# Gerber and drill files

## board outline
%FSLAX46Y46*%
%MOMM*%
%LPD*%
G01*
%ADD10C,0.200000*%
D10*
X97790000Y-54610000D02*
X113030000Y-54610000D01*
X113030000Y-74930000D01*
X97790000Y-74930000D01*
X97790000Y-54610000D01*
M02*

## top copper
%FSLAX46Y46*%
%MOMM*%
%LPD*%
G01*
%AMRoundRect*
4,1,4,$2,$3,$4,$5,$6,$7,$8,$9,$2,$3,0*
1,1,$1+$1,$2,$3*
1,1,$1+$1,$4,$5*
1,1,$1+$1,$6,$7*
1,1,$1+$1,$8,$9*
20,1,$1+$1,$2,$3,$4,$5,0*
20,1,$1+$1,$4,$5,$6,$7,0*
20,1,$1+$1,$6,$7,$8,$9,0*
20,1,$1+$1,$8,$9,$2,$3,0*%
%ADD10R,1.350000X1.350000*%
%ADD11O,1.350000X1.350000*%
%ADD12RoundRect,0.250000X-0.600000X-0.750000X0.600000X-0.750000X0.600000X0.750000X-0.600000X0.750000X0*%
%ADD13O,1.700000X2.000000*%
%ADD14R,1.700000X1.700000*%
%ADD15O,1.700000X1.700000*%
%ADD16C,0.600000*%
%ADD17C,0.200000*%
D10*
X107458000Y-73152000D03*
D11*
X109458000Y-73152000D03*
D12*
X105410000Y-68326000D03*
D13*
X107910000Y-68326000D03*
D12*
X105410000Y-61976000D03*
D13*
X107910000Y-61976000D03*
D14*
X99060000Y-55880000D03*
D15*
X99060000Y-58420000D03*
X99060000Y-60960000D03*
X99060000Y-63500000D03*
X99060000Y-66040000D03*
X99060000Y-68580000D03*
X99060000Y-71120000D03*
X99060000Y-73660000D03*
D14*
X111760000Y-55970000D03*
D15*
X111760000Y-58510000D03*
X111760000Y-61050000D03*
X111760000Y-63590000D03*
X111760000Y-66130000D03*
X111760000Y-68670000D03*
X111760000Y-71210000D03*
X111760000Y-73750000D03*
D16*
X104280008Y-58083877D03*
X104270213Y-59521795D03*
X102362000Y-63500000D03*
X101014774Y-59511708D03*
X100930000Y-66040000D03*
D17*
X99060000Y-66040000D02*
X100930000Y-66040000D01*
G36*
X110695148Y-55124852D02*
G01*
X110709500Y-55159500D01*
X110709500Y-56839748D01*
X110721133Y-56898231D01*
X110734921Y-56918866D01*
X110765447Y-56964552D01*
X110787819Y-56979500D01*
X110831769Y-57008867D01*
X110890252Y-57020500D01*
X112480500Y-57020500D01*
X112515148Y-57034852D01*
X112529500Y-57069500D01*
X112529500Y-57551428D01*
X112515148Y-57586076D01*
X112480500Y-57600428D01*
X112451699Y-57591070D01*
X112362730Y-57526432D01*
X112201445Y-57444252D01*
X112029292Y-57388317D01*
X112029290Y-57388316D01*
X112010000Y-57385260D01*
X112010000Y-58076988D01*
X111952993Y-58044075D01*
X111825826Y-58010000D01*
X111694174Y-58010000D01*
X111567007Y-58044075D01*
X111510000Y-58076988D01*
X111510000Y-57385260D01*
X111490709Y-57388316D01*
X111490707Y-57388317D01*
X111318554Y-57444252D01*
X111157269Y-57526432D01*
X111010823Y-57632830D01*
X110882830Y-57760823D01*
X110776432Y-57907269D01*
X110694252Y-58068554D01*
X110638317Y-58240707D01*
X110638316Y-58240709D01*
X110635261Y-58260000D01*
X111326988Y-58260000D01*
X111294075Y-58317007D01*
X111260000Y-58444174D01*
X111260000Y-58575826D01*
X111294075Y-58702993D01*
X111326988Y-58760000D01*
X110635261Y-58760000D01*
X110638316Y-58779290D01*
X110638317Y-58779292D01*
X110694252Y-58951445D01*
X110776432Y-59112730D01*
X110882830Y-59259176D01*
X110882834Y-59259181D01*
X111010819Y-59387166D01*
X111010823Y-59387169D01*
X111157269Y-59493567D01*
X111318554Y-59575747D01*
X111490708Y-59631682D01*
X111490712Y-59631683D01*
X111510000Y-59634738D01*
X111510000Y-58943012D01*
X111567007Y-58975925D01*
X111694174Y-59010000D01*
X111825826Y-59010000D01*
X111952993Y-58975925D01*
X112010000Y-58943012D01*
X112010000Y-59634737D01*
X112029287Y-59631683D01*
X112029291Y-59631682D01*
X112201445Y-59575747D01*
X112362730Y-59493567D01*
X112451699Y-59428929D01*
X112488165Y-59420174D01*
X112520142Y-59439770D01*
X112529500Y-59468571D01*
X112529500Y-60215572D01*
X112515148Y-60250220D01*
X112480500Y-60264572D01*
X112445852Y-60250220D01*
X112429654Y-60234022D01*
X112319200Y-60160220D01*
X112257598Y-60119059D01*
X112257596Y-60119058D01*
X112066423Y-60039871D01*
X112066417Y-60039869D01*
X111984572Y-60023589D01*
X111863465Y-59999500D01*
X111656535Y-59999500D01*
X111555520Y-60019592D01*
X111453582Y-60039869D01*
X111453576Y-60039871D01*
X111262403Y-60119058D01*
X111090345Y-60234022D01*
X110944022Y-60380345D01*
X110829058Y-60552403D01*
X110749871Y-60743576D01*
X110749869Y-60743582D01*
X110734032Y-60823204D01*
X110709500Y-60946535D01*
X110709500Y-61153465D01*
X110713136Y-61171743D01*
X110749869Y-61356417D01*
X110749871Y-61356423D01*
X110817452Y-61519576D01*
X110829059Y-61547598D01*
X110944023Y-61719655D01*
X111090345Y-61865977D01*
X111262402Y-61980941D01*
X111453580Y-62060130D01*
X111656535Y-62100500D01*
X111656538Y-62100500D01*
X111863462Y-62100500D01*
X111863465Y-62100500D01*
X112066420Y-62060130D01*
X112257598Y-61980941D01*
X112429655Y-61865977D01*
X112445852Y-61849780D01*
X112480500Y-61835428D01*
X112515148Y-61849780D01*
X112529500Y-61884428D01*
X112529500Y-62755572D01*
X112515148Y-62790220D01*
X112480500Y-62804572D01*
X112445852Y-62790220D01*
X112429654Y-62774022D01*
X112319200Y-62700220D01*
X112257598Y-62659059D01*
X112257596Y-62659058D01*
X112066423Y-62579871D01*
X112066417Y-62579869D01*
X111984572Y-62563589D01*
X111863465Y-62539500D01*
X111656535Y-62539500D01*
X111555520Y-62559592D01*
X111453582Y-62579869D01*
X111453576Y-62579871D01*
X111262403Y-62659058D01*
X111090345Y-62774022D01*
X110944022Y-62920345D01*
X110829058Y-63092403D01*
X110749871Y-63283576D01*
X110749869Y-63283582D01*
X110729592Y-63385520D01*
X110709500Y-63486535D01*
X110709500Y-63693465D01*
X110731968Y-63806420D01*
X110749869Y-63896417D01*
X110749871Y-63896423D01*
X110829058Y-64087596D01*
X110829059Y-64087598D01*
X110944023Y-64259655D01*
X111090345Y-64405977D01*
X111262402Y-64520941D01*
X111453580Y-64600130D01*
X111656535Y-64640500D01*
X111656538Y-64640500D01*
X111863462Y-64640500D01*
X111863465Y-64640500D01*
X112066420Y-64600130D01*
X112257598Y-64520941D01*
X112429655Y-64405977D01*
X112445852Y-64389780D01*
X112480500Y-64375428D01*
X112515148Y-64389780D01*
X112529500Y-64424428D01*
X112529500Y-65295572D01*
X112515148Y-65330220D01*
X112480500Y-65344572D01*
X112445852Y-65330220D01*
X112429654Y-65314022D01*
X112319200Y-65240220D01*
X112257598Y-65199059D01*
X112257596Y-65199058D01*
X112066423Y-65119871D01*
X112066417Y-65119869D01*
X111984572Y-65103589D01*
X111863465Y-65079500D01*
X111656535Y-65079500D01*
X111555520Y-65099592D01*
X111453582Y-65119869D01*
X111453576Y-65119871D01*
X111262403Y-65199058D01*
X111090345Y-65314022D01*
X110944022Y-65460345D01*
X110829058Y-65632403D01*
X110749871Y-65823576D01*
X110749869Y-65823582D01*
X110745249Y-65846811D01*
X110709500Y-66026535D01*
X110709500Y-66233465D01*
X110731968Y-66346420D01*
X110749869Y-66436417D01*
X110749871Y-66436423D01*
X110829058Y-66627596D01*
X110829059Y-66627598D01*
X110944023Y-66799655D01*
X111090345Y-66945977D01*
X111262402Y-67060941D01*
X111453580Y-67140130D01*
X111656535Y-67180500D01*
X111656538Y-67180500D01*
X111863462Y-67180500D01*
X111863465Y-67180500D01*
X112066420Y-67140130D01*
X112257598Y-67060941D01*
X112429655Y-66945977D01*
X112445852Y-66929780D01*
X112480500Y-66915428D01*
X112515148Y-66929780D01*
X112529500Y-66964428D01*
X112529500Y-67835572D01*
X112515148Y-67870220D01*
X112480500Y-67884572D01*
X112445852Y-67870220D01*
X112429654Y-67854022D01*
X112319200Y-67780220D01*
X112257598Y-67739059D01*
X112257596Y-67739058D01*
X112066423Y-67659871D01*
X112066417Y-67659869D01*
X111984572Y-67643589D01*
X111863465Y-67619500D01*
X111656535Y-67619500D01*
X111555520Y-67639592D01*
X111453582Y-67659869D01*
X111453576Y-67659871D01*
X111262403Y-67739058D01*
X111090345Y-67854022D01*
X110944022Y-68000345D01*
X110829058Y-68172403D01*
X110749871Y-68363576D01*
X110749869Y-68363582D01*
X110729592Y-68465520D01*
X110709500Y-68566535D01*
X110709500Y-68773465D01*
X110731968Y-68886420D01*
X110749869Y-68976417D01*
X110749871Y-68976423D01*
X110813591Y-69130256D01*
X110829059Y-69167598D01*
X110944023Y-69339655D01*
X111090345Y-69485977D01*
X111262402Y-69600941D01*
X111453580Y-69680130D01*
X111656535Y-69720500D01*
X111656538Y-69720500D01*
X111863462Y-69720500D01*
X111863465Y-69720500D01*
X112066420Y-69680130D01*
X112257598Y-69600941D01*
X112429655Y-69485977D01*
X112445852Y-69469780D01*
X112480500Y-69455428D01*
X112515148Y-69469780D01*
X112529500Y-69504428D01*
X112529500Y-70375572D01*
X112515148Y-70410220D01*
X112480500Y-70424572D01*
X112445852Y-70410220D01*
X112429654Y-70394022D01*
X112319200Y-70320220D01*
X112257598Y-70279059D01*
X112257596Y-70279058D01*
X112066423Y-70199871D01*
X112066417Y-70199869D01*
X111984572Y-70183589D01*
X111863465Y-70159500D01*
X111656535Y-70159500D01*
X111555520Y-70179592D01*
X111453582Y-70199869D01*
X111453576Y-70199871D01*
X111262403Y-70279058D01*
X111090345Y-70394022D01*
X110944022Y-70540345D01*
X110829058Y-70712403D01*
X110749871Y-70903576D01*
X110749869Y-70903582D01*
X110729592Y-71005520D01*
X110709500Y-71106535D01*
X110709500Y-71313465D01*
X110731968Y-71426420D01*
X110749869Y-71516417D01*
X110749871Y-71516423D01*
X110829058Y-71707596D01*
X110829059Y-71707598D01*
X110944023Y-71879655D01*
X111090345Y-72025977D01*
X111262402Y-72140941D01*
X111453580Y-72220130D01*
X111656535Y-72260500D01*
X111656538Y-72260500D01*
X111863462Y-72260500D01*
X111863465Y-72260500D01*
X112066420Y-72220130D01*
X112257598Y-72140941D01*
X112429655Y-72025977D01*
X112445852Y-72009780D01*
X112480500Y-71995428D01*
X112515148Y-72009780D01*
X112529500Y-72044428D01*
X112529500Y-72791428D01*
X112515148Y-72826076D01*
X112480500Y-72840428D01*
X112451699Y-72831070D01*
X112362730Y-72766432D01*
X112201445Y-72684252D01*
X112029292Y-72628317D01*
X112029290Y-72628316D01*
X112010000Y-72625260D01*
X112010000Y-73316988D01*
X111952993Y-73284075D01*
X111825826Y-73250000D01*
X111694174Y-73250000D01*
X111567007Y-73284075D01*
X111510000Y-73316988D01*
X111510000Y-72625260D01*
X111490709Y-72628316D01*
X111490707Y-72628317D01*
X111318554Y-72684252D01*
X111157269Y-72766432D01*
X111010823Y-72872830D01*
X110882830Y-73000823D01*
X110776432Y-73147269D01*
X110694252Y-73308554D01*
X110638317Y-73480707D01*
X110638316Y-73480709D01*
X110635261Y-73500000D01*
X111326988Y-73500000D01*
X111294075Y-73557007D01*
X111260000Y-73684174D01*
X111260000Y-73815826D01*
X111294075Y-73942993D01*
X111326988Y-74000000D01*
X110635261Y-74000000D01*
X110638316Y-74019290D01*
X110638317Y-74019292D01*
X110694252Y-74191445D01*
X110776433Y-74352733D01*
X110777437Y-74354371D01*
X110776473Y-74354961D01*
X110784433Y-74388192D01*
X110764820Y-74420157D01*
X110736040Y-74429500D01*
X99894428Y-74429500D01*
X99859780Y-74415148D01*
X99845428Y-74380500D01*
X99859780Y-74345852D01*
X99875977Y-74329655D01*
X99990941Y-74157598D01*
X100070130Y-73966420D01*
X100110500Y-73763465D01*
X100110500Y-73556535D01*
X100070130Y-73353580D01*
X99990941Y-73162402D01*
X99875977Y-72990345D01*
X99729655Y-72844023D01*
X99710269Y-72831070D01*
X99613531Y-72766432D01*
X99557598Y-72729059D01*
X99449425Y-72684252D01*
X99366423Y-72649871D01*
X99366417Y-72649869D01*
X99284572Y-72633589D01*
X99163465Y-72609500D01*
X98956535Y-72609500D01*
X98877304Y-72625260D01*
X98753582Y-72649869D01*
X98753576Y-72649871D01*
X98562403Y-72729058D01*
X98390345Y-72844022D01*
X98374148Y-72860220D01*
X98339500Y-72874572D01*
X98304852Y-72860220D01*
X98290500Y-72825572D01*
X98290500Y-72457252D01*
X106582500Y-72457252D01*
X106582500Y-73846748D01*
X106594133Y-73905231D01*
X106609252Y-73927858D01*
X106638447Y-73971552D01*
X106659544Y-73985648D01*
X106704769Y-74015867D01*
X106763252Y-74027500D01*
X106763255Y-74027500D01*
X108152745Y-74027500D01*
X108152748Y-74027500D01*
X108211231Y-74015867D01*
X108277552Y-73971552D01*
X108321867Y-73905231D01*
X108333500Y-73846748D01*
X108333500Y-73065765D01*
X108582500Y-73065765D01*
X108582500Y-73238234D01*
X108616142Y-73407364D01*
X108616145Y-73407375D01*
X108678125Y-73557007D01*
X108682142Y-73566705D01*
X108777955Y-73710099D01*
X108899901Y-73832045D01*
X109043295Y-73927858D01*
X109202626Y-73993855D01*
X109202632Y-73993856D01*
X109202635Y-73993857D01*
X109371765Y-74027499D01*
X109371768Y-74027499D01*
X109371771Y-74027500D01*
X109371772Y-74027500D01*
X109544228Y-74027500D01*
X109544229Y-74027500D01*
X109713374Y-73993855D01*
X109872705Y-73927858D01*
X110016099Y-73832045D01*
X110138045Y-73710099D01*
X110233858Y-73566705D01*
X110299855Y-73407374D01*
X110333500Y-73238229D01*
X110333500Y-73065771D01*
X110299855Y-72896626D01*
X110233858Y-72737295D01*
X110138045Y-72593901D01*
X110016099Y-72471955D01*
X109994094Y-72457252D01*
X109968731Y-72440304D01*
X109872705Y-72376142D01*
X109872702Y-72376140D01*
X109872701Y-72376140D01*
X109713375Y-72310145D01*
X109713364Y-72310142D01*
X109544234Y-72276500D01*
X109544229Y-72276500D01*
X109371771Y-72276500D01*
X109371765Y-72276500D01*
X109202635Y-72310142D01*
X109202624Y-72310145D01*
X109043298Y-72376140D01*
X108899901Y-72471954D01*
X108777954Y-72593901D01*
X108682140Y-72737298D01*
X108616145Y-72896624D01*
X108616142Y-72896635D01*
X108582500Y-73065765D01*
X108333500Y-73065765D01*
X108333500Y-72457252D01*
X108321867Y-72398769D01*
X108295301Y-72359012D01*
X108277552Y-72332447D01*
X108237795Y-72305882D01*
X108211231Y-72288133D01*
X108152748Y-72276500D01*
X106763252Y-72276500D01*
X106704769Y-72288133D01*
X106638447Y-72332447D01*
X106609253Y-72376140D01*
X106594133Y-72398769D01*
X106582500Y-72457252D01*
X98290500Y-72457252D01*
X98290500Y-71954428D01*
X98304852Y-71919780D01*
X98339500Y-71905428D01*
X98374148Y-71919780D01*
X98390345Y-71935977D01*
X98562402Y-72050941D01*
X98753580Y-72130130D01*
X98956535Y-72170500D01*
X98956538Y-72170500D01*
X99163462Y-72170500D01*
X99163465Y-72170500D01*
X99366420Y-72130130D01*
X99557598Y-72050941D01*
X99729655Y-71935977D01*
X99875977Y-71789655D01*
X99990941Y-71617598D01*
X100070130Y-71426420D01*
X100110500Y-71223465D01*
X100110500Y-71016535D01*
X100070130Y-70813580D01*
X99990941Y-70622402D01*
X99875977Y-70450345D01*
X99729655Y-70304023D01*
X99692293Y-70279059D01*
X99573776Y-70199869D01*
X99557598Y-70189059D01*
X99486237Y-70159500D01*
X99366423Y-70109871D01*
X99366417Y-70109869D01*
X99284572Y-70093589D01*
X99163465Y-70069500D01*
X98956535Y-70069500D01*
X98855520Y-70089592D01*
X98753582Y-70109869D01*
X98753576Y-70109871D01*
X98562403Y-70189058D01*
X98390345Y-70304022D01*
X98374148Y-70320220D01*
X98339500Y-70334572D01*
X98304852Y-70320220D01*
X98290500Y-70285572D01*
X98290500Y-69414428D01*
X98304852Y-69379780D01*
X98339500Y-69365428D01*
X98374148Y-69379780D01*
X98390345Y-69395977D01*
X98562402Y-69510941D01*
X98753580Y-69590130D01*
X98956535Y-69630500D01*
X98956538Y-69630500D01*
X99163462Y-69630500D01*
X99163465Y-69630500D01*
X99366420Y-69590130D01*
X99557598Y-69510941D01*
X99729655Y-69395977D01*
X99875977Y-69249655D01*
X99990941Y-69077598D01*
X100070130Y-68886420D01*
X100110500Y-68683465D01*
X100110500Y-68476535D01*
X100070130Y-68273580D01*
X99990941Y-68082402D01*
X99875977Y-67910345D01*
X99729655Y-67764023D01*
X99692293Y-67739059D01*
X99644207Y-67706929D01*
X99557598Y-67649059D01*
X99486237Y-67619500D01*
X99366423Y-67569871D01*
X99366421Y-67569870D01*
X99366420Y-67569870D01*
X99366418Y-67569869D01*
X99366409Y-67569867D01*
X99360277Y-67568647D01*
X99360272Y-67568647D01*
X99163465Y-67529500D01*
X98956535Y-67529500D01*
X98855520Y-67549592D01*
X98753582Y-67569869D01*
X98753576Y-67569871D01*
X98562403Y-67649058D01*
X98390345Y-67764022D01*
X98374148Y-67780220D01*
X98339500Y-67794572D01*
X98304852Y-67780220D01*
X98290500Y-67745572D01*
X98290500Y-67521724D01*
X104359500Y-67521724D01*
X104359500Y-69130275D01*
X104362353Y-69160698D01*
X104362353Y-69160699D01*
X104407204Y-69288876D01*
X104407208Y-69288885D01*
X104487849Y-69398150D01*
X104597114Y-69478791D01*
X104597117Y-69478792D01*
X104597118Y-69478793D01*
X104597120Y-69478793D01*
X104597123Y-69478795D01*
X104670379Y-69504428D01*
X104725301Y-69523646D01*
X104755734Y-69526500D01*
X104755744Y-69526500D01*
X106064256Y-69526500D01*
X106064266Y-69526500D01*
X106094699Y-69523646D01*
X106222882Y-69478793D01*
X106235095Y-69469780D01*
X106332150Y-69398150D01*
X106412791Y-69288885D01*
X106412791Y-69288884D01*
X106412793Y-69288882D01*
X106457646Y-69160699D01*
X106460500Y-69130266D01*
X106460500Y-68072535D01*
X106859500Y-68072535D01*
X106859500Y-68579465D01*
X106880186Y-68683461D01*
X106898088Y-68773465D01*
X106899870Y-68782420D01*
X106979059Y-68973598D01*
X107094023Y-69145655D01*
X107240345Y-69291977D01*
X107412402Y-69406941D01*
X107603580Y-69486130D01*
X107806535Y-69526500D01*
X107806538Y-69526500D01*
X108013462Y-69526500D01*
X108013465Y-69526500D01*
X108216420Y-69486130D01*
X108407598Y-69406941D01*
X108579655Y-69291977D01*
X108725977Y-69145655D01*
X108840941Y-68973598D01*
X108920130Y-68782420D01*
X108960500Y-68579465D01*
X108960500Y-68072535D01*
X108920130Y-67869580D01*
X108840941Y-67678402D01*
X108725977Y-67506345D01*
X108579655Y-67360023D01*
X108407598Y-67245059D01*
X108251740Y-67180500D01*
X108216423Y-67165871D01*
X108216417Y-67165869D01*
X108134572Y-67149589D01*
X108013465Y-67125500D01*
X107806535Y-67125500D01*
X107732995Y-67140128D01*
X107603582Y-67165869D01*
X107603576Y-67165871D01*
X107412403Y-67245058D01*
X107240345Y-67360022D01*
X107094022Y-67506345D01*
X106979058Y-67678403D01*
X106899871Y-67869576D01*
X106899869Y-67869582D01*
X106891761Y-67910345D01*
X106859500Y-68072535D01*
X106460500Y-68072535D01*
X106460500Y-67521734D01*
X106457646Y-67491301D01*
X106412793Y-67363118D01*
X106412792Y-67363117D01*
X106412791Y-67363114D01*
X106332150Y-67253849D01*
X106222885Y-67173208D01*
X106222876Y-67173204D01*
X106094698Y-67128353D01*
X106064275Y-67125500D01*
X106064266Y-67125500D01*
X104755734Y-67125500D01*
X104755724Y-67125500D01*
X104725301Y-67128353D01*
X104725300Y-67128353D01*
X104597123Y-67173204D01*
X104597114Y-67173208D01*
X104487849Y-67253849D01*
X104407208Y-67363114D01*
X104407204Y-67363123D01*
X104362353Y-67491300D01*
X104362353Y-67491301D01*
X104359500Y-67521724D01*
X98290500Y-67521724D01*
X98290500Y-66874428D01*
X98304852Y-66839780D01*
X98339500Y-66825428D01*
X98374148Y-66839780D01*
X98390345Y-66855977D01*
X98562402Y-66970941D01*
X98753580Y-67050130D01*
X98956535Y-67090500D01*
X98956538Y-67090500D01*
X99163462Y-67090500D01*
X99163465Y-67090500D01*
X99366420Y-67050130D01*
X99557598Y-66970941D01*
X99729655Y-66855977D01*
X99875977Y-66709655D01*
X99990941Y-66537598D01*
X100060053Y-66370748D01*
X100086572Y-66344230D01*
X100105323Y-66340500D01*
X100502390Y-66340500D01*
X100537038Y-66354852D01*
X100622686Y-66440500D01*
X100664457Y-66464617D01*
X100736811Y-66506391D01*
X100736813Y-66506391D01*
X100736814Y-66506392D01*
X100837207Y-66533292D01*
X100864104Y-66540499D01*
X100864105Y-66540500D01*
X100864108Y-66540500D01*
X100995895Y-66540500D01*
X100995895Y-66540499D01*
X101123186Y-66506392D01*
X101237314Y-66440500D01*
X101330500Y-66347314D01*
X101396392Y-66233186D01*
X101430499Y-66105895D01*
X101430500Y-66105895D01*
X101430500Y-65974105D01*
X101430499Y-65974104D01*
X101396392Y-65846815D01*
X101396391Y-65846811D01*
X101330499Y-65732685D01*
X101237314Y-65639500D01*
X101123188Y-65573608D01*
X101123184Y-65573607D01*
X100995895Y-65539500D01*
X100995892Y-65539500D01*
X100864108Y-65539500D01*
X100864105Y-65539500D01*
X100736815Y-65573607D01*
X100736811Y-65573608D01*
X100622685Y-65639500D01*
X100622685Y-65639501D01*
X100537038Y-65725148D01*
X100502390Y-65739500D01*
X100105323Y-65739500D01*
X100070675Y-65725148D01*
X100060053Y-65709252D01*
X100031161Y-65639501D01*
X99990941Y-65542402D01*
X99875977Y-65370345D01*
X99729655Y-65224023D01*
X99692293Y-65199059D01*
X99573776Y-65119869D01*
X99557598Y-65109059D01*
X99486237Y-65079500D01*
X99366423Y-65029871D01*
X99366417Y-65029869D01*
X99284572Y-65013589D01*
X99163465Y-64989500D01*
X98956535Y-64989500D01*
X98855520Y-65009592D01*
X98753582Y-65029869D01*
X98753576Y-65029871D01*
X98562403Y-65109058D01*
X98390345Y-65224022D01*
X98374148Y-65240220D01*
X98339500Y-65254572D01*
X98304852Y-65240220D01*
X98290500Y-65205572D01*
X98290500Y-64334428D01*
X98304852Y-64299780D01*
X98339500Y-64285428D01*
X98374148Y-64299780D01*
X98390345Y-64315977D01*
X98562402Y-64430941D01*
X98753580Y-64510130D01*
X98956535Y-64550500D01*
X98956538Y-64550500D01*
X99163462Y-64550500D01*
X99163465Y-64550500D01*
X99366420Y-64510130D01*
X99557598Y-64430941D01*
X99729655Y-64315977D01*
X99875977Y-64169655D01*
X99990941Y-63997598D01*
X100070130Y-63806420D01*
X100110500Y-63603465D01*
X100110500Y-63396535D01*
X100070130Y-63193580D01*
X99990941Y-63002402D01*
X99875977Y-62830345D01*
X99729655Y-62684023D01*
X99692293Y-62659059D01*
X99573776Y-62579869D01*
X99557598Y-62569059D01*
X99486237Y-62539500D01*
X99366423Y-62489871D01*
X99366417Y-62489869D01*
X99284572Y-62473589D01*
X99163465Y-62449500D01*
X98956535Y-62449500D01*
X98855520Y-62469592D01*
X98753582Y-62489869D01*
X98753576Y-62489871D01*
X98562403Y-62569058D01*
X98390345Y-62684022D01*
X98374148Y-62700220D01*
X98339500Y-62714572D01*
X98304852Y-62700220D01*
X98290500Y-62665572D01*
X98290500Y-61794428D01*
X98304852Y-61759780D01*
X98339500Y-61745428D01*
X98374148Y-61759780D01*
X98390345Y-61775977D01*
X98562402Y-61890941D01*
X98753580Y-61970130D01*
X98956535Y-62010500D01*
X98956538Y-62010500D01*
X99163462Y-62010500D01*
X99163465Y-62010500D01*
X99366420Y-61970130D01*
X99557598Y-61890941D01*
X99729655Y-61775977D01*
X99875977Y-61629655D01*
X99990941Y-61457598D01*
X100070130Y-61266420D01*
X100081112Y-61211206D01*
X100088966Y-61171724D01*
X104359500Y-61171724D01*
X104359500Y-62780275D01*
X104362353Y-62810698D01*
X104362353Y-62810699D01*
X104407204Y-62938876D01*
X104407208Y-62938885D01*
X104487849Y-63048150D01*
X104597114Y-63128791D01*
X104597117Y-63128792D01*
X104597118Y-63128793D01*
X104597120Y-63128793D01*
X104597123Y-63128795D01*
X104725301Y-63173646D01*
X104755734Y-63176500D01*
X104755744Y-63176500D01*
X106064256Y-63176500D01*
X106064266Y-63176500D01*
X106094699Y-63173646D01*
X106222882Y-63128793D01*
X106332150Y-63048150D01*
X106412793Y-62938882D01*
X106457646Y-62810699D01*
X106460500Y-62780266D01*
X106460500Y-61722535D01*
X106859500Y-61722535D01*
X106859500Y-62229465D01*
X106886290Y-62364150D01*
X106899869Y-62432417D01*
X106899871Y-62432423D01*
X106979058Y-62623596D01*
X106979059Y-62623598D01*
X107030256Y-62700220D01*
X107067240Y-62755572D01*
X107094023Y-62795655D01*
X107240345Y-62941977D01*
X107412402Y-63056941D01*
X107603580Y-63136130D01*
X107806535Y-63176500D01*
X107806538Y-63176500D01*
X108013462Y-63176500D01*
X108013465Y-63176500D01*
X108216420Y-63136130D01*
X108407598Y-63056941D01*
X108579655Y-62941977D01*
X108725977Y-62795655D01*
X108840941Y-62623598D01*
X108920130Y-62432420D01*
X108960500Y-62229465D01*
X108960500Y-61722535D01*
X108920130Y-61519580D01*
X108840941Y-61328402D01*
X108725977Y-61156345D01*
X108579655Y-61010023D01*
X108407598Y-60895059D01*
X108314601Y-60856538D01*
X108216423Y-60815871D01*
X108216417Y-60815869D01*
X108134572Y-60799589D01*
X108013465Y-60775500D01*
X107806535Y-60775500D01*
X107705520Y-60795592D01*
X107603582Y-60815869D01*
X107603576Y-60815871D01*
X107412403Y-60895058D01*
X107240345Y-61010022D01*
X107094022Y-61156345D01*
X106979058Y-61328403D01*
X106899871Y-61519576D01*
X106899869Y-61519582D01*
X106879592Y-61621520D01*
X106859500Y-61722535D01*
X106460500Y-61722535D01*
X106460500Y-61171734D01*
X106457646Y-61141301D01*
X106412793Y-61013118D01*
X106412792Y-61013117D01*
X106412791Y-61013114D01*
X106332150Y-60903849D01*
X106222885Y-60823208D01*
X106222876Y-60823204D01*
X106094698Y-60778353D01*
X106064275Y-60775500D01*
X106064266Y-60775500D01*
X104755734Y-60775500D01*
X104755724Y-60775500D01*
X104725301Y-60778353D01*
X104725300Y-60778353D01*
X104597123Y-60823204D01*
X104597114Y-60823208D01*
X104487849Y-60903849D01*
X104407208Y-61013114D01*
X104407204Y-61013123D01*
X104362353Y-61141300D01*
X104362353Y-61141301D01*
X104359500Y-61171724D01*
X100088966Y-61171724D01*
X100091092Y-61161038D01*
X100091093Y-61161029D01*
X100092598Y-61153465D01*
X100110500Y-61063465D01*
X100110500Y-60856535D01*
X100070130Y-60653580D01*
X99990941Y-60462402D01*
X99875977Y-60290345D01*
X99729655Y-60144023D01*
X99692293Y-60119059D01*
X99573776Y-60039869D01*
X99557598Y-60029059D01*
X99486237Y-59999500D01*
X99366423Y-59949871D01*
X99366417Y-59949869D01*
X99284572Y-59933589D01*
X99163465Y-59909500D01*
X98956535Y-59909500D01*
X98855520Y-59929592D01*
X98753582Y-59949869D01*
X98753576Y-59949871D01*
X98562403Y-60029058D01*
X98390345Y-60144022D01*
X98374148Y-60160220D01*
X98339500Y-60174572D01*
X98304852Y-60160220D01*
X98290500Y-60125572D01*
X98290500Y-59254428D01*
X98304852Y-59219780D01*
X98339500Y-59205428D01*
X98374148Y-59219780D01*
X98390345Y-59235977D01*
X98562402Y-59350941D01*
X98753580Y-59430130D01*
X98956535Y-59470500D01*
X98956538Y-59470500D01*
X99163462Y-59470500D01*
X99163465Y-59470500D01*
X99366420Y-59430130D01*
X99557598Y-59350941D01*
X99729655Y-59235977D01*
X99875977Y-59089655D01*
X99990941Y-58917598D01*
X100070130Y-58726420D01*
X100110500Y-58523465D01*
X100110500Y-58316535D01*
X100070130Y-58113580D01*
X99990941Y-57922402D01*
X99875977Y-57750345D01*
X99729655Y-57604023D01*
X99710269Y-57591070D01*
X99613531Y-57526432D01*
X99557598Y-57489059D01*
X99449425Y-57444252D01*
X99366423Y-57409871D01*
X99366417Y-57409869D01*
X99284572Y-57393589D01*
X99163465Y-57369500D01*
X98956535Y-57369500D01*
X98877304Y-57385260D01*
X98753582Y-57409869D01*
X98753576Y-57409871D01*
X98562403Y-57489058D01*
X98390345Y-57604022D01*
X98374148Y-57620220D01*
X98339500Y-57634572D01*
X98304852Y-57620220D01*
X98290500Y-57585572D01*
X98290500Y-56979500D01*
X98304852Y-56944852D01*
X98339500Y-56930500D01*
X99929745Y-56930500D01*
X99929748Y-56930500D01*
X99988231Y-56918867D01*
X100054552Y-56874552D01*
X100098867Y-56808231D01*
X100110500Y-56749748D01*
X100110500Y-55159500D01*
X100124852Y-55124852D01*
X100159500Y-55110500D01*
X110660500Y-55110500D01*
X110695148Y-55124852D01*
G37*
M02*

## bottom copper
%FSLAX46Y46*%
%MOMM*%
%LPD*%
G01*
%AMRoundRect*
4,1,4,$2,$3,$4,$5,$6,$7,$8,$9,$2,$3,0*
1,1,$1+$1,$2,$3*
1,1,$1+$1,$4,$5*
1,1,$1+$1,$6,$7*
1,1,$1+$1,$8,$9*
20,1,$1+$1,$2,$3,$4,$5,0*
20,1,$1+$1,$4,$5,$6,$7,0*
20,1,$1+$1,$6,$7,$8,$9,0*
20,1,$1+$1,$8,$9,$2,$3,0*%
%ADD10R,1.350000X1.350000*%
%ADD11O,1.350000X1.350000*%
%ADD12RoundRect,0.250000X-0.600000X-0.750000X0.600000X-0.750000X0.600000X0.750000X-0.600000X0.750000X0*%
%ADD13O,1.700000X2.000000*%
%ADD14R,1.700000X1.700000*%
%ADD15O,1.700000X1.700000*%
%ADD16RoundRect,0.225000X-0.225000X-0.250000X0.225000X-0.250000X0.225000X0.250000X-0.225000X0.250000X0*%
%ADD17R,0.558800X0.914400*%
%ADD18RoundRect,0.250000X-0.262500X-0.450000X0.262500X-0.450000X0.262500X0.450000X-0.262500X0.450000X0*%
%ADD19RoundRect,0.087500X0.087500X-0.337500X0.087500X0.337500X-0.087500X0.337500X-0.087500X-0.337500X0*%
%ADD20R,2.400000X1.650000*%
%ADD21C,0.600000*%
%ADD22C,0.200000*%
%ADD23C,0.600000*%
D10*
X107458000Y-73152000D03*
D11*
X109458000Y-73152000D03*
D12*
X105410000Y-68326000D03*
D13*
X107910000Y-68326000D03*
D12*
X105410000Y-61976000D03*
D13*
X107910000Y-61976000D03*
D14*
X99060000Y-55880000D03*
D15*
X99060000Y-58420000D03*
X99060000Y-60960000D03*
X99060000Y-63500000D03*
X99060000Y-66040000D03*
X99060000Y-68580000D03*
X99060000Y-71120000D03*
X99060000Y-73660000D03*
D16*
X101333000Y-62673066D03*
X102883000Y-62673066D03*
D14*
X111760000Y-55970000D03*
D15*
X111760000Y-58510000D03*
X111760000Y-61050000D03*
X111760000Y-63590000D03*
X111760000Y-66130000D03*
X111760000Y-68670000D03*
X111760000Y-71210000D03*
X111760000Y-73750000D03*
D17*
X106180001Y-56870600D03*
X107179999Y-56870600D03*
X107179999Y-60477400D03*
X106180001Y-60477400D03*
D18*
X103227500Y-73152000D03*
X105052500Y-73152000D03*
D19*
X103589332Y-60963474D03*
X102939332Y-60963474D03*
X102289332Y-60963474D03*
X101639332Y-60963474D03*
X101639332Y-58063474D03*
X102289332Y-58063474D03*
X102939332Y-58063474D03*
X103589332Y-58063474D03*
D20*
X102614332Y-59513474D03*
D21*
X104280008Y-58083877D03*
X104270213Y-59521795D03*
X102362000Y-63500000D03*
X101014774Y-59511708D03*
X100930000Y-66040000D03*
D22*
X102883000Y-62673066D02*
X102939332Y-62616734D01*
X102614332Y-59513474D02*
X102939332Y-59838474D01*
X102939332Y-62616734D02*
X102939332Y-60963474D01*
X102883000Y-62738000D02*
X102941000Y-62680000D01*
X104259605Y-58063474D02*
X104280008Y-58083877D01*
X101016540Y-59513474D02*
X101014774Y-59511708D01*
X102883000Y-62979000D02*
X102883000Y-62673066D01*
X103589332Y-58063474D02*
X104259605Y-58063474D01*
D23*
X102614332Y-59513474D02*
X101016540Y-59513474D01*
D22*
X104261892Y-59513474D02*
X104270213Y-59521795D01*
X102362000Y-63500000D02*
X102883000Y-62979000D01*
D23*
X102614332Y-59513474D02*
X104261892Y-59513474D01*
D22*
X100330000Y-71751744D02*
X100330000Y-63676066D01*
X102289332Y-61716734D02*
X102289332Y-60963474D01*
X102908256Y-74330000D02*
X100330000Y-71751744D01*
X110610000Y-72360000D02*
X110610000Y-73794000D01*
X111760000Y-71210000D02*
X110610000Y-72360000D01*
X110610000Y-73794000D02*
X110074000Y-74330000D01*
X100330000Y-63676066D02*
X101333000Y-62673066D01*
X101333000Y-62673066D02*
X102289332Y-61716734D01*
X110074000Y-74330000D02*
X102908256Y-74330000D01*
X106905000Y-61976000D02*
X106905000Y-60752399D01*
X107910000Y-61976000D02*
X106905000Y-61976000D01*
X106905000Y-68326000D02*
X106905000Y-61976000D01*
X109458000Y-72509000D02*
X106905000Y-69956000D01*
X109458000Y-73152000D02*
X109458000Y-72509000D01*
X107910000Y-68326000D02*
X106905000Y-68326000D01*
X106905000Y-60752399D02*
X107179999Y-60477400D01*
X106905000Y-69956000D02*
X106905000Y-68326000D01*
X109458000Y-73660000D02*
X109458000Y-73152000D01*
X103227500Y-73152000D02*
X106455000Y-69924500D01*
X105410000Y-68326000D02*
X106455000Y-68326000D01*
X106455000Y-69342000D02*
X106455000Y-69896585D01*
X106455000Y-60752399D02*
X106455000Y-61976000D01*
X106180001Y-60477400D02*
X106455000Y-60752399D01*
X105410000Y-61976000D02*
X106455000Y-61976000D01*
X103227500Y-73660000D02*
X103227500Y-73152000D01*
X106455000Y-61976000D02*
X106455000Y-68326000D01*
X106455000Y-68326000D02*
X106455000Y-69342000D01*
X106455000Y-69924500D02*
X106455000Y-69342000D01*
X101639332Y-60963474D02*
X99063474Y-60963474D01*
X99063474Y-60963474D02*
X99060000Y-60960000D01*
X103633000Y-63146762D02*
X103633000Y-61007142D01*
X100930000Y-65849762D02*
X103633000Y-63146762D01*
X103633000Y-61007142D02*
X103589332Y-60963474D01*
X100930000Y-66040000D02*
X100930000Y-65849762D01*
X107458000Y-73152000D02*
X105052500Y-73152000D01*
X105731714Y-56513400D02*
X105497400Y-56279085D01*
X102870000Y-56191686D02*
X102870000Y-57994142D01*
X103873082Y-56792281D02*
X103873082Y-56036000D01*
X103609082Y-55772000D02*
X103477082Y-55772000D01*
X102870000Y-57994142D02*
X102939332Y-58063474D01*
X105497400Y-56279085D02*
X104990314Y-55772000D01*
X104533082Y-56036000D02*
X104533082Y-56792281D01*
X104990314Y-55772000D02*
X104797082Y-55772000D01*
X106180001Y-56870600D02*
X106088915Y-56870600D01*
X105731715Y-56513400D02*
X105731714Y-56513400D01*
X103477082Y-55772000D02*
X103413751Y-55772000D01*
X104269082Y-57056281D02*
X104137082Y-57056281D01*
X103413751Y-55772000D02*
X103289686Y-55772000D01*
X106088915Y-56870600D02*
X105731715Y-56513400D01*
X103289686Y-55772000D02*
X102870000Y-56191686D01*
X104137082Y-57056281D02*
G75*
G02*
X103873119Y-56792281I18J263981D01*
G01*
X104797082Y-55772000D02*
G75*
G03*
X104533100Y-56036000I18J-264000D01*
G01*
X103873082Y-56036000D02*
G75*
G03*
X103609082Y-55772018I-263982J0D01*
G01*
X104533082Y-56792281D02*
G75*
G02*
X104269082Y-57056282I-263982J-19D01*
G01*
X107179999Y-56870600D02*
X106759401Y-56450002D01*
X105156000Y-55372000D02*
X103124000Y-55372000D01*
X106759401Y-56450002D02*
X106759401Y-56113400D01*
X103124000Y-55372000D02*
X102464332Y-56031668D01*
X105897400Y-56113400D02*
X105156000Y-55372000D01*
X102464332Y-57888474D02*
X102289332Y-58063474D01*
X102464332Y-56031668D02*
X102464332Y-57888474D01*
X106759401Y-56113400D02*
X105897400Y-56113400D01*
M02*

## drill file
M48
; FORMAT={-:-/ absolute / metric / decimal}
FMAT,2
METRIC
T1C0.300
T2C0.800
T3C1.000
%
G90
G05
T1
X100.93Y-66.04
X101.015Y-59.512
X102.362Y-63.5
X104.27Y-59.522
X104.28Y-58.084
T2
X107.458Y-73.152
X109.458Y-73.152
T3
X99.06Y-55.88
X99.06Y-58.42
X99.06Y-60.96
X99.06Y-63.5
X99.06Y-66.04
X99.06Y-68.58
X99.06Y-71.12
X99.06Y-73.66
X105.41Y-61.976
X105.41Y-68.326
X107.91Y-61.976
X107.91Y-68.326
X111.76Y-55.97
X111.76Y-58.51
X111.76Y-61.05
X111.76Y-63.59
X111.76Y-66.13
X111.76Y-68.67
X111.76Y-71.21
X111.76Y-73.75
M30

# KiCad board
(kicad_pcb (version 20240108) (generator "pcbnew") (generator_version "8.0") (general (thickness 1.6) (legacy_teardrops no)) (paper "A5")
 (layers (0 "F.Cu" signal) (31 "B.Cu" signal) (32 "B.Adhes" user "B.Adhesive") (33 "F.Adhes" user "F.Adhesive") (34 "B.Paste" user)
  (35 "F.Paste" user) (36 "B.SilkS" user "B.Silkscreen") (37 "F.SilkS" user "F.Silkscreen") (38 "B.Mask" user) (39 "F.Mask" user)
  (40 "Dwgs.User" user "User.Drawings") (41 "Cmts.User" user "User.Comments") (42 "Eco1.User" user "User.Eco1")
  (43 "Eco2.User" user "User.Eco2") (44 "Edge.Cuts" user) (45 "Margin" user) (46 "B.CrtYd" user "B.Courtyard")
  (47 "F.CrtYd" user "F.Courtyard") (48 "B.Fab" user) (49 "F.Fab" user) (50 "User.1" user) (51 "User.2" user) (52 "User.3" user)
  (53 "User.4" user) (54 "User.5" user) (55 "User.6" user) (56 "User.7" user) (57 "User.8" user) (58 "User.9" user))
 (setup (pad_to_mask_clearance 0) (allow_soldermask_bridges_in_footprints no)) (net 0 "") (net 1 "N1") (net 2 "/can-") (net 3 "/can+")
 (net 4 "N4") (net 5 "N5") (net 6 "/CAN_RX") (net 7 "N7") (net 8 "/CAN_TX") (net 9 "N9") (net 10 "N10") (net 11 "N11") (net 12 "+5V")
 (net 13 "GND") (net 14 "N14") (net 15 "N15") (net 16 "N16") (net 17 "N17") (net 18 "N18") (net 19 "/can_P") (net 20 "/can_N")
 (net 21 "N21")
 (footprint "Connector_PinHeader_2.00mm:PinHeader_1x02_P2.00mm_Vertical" (layer "F.Cu") (at 107.458 73.152 90)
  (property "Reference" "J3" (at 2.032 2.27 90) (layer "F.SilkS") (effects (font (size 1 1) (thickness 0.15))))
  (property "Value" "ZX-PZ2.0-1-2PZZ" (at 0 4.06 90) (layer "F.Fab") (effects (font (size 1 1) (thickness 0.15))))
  (pad "1" thru_hole rect (at 0 0 90) (size 1.35 1.35) (drill 0.8) (layers "*.Cu" "*.Mask") (remove_unused_layers no) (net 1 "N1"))
  (pad "2" thru_hole oval (at 0 2 90) (size 1.35 1.35) (drill 0.8) (layers "*.Cu" "*.Mask") (remove_unused_layers no) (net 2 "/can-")))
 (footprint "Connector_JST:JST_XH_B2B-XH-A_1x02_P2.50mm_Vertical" (layer "F.Cu") (at 105.41 68.326)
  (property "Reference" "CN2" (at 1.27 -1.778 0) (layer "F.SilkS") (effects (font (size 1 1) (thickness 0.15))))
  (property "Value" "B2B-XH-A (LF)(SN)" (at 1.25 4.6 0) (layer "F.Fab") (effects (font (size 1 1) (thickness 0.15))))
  (pad "1" thru_hole roundrect (at 0 0) (size 1.7 2) (drill 1) (layers "*.Cu" "*.Mask") (remove_unused_layers no)
   (roundrect_rratio 0.147059) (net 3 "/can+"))
  (pad "2" thru_hole oval (at 2.5 0) (size 1.7 2) (drill 1) (layers "*.Cu" "*.Mask") (remove_unused_layers no) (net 2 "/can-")))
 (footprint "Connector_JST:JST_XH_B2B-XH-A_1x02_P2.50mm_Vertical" (layer "F.Cu") (at 105.41 61.976)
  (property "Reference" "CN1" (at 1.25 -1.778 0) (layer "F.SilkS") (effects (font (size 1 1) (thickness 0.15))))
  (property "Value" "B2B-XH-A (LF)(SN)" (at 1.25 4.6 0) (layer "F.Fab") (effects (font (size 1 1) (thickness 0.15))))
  (pad "1" thru_hole roundrect (at 0 0) (size 1.7 2) (drill 1) (layers "*.Cu" "*.Mask") (remove_unused_layers no)
   (roundrect_rratio 0.147059) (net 3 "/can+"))
  (pad "2" thru_hole oval (at 2.5 0) (size 1.7 2) (drill 1) (layers "*.Cu" "*.Mask") (remove_unused_layers no) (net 2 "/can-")))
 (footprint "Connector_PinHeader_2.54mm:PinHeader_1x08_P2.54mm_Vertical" (layer "B.Cu") (at 99.06 55.88 180)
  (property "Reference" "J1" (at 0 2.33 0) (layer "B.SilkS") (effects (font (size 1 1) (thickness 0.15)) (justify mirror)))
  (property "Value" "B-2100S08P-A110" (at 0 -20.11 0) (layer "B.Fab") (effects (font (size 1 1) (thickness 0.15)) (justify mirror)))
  (pad "1" thru_hole rect (at 0 0 180) (size 1.7 1.7) (drill 1) (layers "*.Cu" "*.Mask") (remove_unused_layers no) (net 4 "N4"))
  (pad "2" thru_hole oval (at 0 -2.54 180) (size 1.7 1.7) (drill 1) (layers "*.Cu" "*.Mask") (remove_unused_layers no) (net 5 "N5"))
  (pad "3" thru_hole oval (at 0 -5.08 180) (size 1.7 1.7) (drill 1) (layers "*.Cu" "*.Mask") (remove_unused_layers no) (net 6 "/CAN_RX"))
  (pad "4" thru_hole oval (at 0 -7.62 180) (size 1.7 1.7) (drill 1) (layers "*.Cu" "*.Mask") (remove_unused_layers no) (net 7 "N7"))
  (pad "5" thru_hole oval (at 0 -10.16 180) (size 1.7 1.7) (drill 1) (layers "*.Cu" "*.Mask") (remove_unused_layers no) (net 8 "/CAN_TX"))
  (pad "6" thru_hole oval (at 0 -12.7 180) (size 1.7 1.7) (drill 1) (layers "*.Cu" "*.Mask") (remove_unused_layers no) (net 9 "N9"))
  (pad "7" thru_hole oval (at 0 -15.24 180) (size 1.7 1.7) (drill 1) (layers "*.Cu" "*.Mask") (remove_unused_layers no) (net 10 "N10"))
  (pad "8" thru_hole oval (at 0 -17.78 180) (size 1.7 1.7) (drill 1) (layers "*.Cu" "*.Mask") (remove_unused_layers no) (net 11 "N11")))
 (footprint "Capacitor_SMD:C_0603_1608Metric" (layer "B.Cu") (at 102.108 62.673066)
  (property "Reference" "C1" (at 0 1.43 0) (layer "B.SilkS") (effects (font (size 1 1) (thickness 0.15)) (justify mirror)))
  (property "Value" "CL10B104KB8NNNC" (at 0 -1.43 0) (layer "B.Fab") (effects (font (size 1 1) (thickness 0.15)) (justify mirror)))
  (pad "1" smd roundrect (at -0.775 0) (size 0.9 0.95) (layers "B.Cu" "B.Paste" "B.Mask") (roundrect_rratio 0.25) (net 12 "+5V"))
  (pad "2" smd roundrect (at 0.775 0) (size 0.9 0.95) (layers "B.Cu" "B.Paste" "B.Mask") (roundrect_rratio 0.25) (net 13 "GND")))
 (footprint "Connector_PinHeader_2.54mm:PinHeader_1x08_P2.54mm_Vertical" (layer "B.Cu") (at 111.76 55.97 180)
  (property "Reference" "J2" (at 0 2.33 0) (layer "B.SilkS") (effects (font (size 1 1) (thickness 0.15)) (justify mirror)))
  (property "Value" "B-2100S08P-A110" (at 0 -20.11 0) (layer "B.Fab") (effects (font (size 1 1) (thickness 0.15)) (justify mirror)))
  (pad "1" thru_hole rect (at 0 0 180) (size 1.7 1.7) (drill 1) (layers "*.Cu" "*.Mask") (remove_unused_layers no) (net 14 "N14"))
  (pad "2" thru_hole oval (at 0 -2.54 180) (size 1.7 1.7) (drill 1) (layers "*.Cu" "*.Mask") (remove_unused_layers no) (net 13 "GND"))
  (pad "3" thru_hole oval (at 0 -5.08 180) (size 1.7 1.7) (drill 1) (layers "*.Cu" "*.Mask") (remove_unused_layers no) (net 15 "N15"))
  (pad "4" thru_hole oval (at 0 -7.62 180) (size 1.7 1.7) (drill 1) (layers "*.Cu" "*.Mask") (remove_unused_layers no) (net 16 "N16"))
  (pad "5" thru_hole oval (at 0 -10.16 180) (size 1.7 1.7) (drill 1) (layers "*.Cu" "*.Mask") (remove_unused_layers no) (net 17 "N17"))
  (pad "6" thru_hole oval (at 0 -12.7 180) (size 1.7 1.7) (drill 1) (layers "*.Cu" "*.Mask") (remove_unused_layers no) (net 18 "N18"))
  (pad "7" thru_hole oval (at 0 -15.24 180) (size 1.7 1.7) (drill 1) (layers "*.Cu" "*.Mask") (remove_unused_layers no) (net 12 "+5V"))
  (pad "8" thru_hole oval (at 0 -17.78 180) (size 1.7 1.7) (drill 1) (layers "*.Cu" "*.Mask") (remove_unused_layers no) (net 13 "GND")))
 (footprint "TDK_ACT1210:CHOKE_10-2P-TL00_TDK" (layer "B.Cu") (at 106.68 58.674 -90)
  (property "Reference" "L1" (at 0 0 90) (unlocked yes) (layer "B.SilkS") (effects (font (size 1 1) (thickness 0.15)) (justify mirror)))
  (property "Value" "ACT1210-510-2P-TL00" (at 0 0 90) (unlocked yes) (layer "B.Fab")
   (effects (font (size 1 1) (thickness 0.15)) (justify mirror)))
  (pad "1" smd rect (at -1.8034 0.499999 270) (size 0.9144 0.5588) (layers "B.Cu" "B.Paste" "B.Mask") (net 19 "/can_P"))
  (pad "2" smd rect (at -1.8034 -0.499999 270) (size 0.9144 0.5588) (layers "B.Cu" "B.Paste" "B.Mask") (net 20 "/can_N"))
  (pad "3" smd rect (at 1.8034 -0.499999 270) (size 0.9144 0.5588) (layers "B.Cu" "B.Paste" "B.Mask") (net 2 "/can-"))
  (pad "4" smd rect (at 1.8034 0.499999 270) (size 0.9144 0.5588) (layers "B.Cu" "B.Paste" "B.Mask") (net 3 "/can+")))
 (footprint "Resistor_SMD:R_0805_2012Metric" (layer "B.Cu") (at 104.14 73.152)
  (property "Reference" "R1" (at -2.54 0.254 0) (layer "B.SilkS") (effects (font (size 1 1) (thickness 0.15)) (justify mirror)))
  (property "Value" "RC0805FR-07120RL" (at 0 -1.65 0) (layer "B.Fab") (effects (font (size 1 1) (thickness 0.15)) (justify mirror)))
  (pad "1" smd roundrect (at -0.9125 0) (size 1.025 1.4) (layers "B.Cu" "B.Paste" "B.Mask") (roundrect_rratio 0.243902) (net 3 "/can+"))
  (pad "2" smd roundrect (at 0.9125 0) (size 1.025 1.4) (layers "B.Cu" "B.Paste" "B.Mask") (roundrect_rratio 0.243902) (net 1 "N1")))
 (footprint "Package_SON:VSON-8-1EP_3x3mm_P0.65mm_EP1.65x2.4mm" (layer "B.Cu") (at 102.614332 59.513474 90)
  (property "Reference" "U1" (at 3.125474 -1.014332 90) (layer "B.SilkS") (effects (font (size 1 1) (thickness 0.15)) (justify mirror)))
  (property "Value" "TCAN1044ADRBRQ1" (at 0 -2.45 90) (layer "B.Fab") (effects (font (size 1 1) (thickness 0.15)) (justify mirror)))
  (pad "" smd roundrect (at 0 0 90) (size 1.33 1.93) (layers "B.Paste") (roundrect_rratio 0.18797))
  (pad "1" smd roundrect (at -1.45 0.975 90) (size 0.85 0.35) (layers "B.Cu" "B.Paste" "B.Mask") (roundrect_rratio 0.25) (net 8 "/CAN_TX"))
  (pad "2" smd roundrect (at -1.45 0.325 90) (size 0.85 0.35) (layers "B.Cu" "B.Paste" "B.Mask") (roundrect_rratio 0.25) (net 13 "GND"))
  (pad "3" smd roundrect (at -1.45 -0.325 90) (size 0.85 0.35) (layers "B.Cu" "B.Paste" "B.Mask") (roundrect_rratio 0.25) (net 12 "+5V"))
  (pad "4" smd roundrect (at -1.45 -0.975 90) (size 0.85 0.35) (layers "B.Cu" "B.Paste" "B.Mask") (roundrect_rratio 0.25) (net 6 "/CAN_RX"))
  (pad "5" smd roundrect (at 1.45 -0.975 90) (size 0.85 0.35) (layers "B.Cu" "B.Paste" "B.Mask") (roundrect_rratio 0.25) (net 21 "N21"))
  (pad "6" smd roundrect (at 1.45 -0.325 90) (size 0.85 0.35) (layers "B.Cu" "B.Paste" "B.Mask") (roundrect_rratio 0.25) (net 20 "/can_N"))
  (pad "7" smd roundrect (at 1.45 0.325 90) (size 0.85 0.35) (layers "B.Cu" "B.Paste" "B.Mask") (roundrect_rratio 0.25) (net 19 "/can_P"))
  (pad "8" smd roundrect (at 1.45 0.975 90) (size 0.85 0.35) (layers "B.Cu" "B.Paste" "B.Mask") (roundrect_rratio 0.25) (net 13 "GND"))
  (pad "9" smd rect (at 0 0 90) (size 1.65 2.4) (layers "B.Cu" "B.Mask") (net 13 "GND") (zone_connect 2)))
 (gr_rect (start 97.79 54.61) (end 113.03 74.93) (stroke (width 0.2) (type default)) (fill none) (layer "Edge.Cuts"))
 (via (at 104.280008 58.083877) (size 0.6) (drill 0.3) (layers "F.Cu" "B.Cu") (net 13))
 (via (at 104.270213 59.521795) (size 0.6) (drill 0.3) (layers "F.Cu" "B.Cu") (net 13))
 (via (at 102.362 63.5) (size 0.6) (drill 0.3) (layers "F.Cu" "B.Cu") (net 13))
 (via (at 101.014774 59.511708) (size 0.6) (drill 0.3) (layers "F.Cu" "B.Cu") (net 13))
 (segment (start 102.883 62.673066) (end 102.939332 62.616734) (width 0.2) (layer "B.Cu") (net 13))
 (segment (start 102.614332 59.513474) (end 102.939332 59.838474) (width 0.2) (layer "B.Cu") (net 13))
 (segment (start 102.939332 62.616734) (end 102.939332 60.963474) (width 0.2) (layer "B.Cu") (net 13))
 (segment (start 102.883 62.738) (end 102.941 62.68) (width 0.2) (layer "B.Cu") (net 13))
 (segment (start 104.259605 58.063474) (end 104.280008 58.083877) (width 0.2) (layer "B.Cu") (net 13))
 (segment (start 101.01654 59.513474) (end 101.014774 59.511708) (width 0.2) (layer "B.Cu") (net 13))
 (segment (start 102.883 62.979) (end 102.883 62.673066) (width 0.2) (layer "B.Cu") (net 13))
 (segment (start 103.589332 58.063474) (end 104.259605 58.063474) (width 0.2) (layer "B.Cu") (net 13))
 (segment (start 102.614332 59.513474) (end 101.01654 59.513474) (width 0.6) (layer "B.Cu") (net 13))
 (segment (start 104.261892 59.513474) (end 104.270213 59.521795) (width 0.2) (layer "B.Cu") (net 13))
 (segment (start 102.362 63.5) (end 102.883 62.979) (width 0.2) (layer "B.Cu") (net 13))
 (segment (start 102.614332 59.513474) (end 104.261892 59.513474) (width 0.6) (layer "B.Cu") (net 13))
 (segment (start 100.33 71.751744) (end 100.33 63.676066) (width 0.2) (layer "B.Cu") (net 12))
 (segment (start 102.289332 61.716734) (end 102.289332 60.963474) (width 0.2) (layer "B.Cu") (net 12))
 (segment (start 102.908256 74.33) (end 100.33 71.751744) (width 0.2) (layer "B.Cu") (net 12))
 (segment (start 110.61 72.36) (end 110.61 73.794) (width 0.2) (layer "B.Cu") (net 12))
 (segment (start 111.76 71.21) (end 110.61 72.36) (width 0.2) (layer "B.Cu") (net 12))
 (segment (start 110.61 73.794) (end 110.074 74.33) (width 0.2) (layer "B.Cu") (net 12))
 (segment (start 100.33 63.676066) (end 101.333 62.673066) (width 0.2) (layer "B.Cu") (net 12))
 (segment (start 101.333 62.673066) (end 102.289332 61.716734) (width 0.2) (layer "B.Cu") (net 12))
 (segment (start 110.074 74.33) (end 102.908256 74.33) (width 0.2) (layer "B.Cu") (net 12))
 (segment (start 106.905 61.976) (end 106.905 60.752399) (width 0.2) (layer "B.Cu") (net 2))
 (segment (start 107.91 61.976) (end 106.905 61.976) (width 0.2) (layer "B.Cu") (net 2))
 (segment (start 106.905 68.326) (end 106.905 61.976) (width 0.2) (layer "B.Cu") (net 2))
 (segment (start 109.458 72.509) (end 106.905 69.956) (width 0.2) (layer "B.Cu") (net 2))
 (segment (start 109.458 73.152) (end 109.458 72.509) (width 0.2) (layer "B.Cu") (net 2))
 (segment (start 107.91 68.326) (end 106.905 68.326) (width 0.2) (layer "B.Cu") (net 2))
 (segment (start 106.905 60.752399) (end 107.179999 60.4774) (width 0.2) (layer "B.Cu") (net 2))
 (segment (start 106.905 69.956) (end 106.905 68.326) (width 0.2) (layer "B.Cu") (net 2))
 (segment (start 109.458 73.66) (end 109.458 73.152) (width 0.2) (layer "B.Cu") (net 2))
 (segment (start 103.2275 73.152) (end 106.455 69.9245) (width 0.2) (layer "B.Cu") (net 3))
 (segment (start 105.41 68.326) (end 106.455 68.326) (width 0.2) (layer "B.Cu") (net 3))
 (segment (start 106.455 69.342) (end 106.455 69.896585) (width 0.2) (layer "B.Cu") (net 3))
 (segment (start 106.455 60.752399) (end 106.455 61.976) (width 0.2) (layer "B.Cu") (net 3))
 (segment (start 106.180001 60.4774) (end 106.455 60.752399) (width 0.2) (layer "B.Cu") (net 3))
 (segment (start 105.41 61.976) (end 106.455 61.976) (width 0.2) (layer "B.Cu") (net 3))
 (segment (start 103.2275 73.66) (end 103.2275 73.152) (width 0.2) (layer "B.Cu") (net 3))
 (segment (start 106.455 61.976) (end 106.455 68.326) (width 0.2) (layer "B.Cu") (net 3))
 (segment (start 106.455 68.326) (end 106.455 69.342) (width 0.2) (layer "B.Cu") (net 3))
 (segment (start 106.455 69.9245) (end 106.455 69.342) (width 0.2) (layer "B.Cu") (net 3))
 (segment (start 101.639332 60.963474) (end 99.063474 60.963474) (width 0.2) (layer "B.Cu") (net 6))
 (segment (start 99.063474 60.963474) (end 99.06 60.96) (width 0.2) (layer "B.Cu") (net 6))
 (segment (start 99.06 66.04) (end 100.93 66.04) (width 0.2) (layer "F.Cu") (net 8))
 (via (at 100.93 66.04) (size 0.6) (drill 0.3) (layers "F.Cu" "B.Cu") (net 8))
 (segment (start 103.633 63.146762) (end 103.633 61.007142) (width 0.2) (layer "B.Cu") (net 8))
 (segment (start 100.93 65.849762) (end 103.633 63.146762) (width 0.2) (layer "B.Cu") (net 8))
 (segment (start 103.633 61.007142) (end 103.589332 60.963474) (width 0.2) (layer "B.Cu") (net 8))
 (segment (start 100.93 66.04) (end 100.93 65.849762) (width 0.2) (layer "B.Cu") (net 8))
 (segment (start 107.458 73.152) (end 105.0525 73.152) (width 0.2) (layer "B.Cu") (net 1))
 (segment (start 105.731714 56.5134) (end 105.4974 56.279085) (width 0.2) (layer "B.Cu") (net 19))
 (segment (start 102.87 56.191686) (end 102.87 57.994142) (width 0.2) (layer "B.Cu") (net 19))
 (segment (start 103.873082 56.792281) (end 103.873082 56.036) (width 0.2) (layer "B.Cu") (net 19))
 (segment (start 103.609082 55.772) (end 103.477082 55.772) (width 0.2) (layer "B.Cu") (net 19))
 (segment (start 102.87 57.994142) (end 102.939332 58.063474) (width 0.2) (layer "B.Cu") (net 19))
 (segment (start 105.4974 56.279085) (end 104.990314 55.772) (width 0.2) (layer "B.Cu") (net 19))
 (segment (start 104.533082 56.036) (end 104.533082 56.792281) (width 0.2) (layer "B.Cu") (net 19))
 (segment (start 104.990314 55.772) (end 104.797082 55.772) (width 0.2) (layer "B.Cu") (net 19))
 (segment (start 106.180001 56.8706) (end 106.088915 56.8706) (width 0.2) (layer "B.Cu") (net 19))
 (segment (start 105.731715 56.5134) (end 105.731714 56.5134) (width 0.2) (layer "B.Cu") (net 19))
 (segment (start 103.477082 55.772) (end 103.413751 55.772) (width 0.2) (layer "B.Cu") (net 19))
 (segment (start 104.269082 57.056281) (end 104.137082 57.056281) (width 0.2) (layer "B.Cu") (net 19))
 (segment (start 103.413751 55.772) (end 103.289686 55.772) (width 0.2) (layer "B.Cu") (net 19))
 (segment (start 106.088915 56.8706) (end 105.731715 56.5134) (width 0.2) (layer "B.Cu") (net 19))
 (segment (start 103.289686 55.772) (end 102.87 56.191686) (width 0.2) (layer "B.Cu") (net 19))
 (arc (start 104.137082 57.056281) (mid 103.950406 56.978957) (end 103.873082 56.792281) (width 0.2) (layer "B.Cu") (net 19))
 (arc (start 104.797082 55.772) (mid 104.610406 55.849324) (end 104.533082 56.036) (width 0.2) (layer "B.Cu") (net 19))
 (arc (start 103.873082 56.036) (mid 103.795758 55.849324) (end 103.609082 55.772) (width 0.2) (layer "B.Cu") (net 19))
 (arc (start 104.533082 56.792281) (mid 104.455758 56.978957) (end 104.269082 57.056281) (width 0.2) (layer "B.Cu") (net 19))
 (segment (start 107.179999 56.8706) (end 106.759401 56.450002) (width 0.2) (layer "B.Cu") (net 20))
 (segment (start 105.156 55.372) (end 103.124 55.372) (width 0.2) (layer "B.Cu") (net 20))
 (segment (start 106.759401 56.450002) (end 106.759401 56.1134) (width 0.2) (layer "B.Cu") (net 20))
 (segment (start 103.124 55.372) (end 102.464332 56.031668) (width 0.2) (layer "B.Cu") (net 20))
 (segment (start 105.8974 56.1134) (end 105.156 55.372) (width 0.2) (layer "B.Cu") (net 20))
 (segment (start 102.464332 57.888474) (end 102.289332 58.063474) (width 0.2) (layer "B.Cu") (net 20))
 (segment (start 102.464332 56.031668) (end 102.464332 57.888474) (width 0.2) (layer "B.Cu") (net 20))
 (segment (start 106.759401 56.1134) (end 105.8974 56.1134) (width 0.2) (layer "B.Cu") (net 20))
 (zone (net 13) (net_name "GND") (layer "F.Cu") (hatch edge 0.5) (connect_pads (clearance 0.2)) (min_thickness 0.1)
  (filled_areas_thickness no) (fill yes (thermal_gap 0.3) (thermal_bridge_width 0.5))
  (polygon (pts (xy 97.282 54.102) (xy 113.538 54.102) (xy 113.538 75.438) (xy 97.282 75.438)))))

